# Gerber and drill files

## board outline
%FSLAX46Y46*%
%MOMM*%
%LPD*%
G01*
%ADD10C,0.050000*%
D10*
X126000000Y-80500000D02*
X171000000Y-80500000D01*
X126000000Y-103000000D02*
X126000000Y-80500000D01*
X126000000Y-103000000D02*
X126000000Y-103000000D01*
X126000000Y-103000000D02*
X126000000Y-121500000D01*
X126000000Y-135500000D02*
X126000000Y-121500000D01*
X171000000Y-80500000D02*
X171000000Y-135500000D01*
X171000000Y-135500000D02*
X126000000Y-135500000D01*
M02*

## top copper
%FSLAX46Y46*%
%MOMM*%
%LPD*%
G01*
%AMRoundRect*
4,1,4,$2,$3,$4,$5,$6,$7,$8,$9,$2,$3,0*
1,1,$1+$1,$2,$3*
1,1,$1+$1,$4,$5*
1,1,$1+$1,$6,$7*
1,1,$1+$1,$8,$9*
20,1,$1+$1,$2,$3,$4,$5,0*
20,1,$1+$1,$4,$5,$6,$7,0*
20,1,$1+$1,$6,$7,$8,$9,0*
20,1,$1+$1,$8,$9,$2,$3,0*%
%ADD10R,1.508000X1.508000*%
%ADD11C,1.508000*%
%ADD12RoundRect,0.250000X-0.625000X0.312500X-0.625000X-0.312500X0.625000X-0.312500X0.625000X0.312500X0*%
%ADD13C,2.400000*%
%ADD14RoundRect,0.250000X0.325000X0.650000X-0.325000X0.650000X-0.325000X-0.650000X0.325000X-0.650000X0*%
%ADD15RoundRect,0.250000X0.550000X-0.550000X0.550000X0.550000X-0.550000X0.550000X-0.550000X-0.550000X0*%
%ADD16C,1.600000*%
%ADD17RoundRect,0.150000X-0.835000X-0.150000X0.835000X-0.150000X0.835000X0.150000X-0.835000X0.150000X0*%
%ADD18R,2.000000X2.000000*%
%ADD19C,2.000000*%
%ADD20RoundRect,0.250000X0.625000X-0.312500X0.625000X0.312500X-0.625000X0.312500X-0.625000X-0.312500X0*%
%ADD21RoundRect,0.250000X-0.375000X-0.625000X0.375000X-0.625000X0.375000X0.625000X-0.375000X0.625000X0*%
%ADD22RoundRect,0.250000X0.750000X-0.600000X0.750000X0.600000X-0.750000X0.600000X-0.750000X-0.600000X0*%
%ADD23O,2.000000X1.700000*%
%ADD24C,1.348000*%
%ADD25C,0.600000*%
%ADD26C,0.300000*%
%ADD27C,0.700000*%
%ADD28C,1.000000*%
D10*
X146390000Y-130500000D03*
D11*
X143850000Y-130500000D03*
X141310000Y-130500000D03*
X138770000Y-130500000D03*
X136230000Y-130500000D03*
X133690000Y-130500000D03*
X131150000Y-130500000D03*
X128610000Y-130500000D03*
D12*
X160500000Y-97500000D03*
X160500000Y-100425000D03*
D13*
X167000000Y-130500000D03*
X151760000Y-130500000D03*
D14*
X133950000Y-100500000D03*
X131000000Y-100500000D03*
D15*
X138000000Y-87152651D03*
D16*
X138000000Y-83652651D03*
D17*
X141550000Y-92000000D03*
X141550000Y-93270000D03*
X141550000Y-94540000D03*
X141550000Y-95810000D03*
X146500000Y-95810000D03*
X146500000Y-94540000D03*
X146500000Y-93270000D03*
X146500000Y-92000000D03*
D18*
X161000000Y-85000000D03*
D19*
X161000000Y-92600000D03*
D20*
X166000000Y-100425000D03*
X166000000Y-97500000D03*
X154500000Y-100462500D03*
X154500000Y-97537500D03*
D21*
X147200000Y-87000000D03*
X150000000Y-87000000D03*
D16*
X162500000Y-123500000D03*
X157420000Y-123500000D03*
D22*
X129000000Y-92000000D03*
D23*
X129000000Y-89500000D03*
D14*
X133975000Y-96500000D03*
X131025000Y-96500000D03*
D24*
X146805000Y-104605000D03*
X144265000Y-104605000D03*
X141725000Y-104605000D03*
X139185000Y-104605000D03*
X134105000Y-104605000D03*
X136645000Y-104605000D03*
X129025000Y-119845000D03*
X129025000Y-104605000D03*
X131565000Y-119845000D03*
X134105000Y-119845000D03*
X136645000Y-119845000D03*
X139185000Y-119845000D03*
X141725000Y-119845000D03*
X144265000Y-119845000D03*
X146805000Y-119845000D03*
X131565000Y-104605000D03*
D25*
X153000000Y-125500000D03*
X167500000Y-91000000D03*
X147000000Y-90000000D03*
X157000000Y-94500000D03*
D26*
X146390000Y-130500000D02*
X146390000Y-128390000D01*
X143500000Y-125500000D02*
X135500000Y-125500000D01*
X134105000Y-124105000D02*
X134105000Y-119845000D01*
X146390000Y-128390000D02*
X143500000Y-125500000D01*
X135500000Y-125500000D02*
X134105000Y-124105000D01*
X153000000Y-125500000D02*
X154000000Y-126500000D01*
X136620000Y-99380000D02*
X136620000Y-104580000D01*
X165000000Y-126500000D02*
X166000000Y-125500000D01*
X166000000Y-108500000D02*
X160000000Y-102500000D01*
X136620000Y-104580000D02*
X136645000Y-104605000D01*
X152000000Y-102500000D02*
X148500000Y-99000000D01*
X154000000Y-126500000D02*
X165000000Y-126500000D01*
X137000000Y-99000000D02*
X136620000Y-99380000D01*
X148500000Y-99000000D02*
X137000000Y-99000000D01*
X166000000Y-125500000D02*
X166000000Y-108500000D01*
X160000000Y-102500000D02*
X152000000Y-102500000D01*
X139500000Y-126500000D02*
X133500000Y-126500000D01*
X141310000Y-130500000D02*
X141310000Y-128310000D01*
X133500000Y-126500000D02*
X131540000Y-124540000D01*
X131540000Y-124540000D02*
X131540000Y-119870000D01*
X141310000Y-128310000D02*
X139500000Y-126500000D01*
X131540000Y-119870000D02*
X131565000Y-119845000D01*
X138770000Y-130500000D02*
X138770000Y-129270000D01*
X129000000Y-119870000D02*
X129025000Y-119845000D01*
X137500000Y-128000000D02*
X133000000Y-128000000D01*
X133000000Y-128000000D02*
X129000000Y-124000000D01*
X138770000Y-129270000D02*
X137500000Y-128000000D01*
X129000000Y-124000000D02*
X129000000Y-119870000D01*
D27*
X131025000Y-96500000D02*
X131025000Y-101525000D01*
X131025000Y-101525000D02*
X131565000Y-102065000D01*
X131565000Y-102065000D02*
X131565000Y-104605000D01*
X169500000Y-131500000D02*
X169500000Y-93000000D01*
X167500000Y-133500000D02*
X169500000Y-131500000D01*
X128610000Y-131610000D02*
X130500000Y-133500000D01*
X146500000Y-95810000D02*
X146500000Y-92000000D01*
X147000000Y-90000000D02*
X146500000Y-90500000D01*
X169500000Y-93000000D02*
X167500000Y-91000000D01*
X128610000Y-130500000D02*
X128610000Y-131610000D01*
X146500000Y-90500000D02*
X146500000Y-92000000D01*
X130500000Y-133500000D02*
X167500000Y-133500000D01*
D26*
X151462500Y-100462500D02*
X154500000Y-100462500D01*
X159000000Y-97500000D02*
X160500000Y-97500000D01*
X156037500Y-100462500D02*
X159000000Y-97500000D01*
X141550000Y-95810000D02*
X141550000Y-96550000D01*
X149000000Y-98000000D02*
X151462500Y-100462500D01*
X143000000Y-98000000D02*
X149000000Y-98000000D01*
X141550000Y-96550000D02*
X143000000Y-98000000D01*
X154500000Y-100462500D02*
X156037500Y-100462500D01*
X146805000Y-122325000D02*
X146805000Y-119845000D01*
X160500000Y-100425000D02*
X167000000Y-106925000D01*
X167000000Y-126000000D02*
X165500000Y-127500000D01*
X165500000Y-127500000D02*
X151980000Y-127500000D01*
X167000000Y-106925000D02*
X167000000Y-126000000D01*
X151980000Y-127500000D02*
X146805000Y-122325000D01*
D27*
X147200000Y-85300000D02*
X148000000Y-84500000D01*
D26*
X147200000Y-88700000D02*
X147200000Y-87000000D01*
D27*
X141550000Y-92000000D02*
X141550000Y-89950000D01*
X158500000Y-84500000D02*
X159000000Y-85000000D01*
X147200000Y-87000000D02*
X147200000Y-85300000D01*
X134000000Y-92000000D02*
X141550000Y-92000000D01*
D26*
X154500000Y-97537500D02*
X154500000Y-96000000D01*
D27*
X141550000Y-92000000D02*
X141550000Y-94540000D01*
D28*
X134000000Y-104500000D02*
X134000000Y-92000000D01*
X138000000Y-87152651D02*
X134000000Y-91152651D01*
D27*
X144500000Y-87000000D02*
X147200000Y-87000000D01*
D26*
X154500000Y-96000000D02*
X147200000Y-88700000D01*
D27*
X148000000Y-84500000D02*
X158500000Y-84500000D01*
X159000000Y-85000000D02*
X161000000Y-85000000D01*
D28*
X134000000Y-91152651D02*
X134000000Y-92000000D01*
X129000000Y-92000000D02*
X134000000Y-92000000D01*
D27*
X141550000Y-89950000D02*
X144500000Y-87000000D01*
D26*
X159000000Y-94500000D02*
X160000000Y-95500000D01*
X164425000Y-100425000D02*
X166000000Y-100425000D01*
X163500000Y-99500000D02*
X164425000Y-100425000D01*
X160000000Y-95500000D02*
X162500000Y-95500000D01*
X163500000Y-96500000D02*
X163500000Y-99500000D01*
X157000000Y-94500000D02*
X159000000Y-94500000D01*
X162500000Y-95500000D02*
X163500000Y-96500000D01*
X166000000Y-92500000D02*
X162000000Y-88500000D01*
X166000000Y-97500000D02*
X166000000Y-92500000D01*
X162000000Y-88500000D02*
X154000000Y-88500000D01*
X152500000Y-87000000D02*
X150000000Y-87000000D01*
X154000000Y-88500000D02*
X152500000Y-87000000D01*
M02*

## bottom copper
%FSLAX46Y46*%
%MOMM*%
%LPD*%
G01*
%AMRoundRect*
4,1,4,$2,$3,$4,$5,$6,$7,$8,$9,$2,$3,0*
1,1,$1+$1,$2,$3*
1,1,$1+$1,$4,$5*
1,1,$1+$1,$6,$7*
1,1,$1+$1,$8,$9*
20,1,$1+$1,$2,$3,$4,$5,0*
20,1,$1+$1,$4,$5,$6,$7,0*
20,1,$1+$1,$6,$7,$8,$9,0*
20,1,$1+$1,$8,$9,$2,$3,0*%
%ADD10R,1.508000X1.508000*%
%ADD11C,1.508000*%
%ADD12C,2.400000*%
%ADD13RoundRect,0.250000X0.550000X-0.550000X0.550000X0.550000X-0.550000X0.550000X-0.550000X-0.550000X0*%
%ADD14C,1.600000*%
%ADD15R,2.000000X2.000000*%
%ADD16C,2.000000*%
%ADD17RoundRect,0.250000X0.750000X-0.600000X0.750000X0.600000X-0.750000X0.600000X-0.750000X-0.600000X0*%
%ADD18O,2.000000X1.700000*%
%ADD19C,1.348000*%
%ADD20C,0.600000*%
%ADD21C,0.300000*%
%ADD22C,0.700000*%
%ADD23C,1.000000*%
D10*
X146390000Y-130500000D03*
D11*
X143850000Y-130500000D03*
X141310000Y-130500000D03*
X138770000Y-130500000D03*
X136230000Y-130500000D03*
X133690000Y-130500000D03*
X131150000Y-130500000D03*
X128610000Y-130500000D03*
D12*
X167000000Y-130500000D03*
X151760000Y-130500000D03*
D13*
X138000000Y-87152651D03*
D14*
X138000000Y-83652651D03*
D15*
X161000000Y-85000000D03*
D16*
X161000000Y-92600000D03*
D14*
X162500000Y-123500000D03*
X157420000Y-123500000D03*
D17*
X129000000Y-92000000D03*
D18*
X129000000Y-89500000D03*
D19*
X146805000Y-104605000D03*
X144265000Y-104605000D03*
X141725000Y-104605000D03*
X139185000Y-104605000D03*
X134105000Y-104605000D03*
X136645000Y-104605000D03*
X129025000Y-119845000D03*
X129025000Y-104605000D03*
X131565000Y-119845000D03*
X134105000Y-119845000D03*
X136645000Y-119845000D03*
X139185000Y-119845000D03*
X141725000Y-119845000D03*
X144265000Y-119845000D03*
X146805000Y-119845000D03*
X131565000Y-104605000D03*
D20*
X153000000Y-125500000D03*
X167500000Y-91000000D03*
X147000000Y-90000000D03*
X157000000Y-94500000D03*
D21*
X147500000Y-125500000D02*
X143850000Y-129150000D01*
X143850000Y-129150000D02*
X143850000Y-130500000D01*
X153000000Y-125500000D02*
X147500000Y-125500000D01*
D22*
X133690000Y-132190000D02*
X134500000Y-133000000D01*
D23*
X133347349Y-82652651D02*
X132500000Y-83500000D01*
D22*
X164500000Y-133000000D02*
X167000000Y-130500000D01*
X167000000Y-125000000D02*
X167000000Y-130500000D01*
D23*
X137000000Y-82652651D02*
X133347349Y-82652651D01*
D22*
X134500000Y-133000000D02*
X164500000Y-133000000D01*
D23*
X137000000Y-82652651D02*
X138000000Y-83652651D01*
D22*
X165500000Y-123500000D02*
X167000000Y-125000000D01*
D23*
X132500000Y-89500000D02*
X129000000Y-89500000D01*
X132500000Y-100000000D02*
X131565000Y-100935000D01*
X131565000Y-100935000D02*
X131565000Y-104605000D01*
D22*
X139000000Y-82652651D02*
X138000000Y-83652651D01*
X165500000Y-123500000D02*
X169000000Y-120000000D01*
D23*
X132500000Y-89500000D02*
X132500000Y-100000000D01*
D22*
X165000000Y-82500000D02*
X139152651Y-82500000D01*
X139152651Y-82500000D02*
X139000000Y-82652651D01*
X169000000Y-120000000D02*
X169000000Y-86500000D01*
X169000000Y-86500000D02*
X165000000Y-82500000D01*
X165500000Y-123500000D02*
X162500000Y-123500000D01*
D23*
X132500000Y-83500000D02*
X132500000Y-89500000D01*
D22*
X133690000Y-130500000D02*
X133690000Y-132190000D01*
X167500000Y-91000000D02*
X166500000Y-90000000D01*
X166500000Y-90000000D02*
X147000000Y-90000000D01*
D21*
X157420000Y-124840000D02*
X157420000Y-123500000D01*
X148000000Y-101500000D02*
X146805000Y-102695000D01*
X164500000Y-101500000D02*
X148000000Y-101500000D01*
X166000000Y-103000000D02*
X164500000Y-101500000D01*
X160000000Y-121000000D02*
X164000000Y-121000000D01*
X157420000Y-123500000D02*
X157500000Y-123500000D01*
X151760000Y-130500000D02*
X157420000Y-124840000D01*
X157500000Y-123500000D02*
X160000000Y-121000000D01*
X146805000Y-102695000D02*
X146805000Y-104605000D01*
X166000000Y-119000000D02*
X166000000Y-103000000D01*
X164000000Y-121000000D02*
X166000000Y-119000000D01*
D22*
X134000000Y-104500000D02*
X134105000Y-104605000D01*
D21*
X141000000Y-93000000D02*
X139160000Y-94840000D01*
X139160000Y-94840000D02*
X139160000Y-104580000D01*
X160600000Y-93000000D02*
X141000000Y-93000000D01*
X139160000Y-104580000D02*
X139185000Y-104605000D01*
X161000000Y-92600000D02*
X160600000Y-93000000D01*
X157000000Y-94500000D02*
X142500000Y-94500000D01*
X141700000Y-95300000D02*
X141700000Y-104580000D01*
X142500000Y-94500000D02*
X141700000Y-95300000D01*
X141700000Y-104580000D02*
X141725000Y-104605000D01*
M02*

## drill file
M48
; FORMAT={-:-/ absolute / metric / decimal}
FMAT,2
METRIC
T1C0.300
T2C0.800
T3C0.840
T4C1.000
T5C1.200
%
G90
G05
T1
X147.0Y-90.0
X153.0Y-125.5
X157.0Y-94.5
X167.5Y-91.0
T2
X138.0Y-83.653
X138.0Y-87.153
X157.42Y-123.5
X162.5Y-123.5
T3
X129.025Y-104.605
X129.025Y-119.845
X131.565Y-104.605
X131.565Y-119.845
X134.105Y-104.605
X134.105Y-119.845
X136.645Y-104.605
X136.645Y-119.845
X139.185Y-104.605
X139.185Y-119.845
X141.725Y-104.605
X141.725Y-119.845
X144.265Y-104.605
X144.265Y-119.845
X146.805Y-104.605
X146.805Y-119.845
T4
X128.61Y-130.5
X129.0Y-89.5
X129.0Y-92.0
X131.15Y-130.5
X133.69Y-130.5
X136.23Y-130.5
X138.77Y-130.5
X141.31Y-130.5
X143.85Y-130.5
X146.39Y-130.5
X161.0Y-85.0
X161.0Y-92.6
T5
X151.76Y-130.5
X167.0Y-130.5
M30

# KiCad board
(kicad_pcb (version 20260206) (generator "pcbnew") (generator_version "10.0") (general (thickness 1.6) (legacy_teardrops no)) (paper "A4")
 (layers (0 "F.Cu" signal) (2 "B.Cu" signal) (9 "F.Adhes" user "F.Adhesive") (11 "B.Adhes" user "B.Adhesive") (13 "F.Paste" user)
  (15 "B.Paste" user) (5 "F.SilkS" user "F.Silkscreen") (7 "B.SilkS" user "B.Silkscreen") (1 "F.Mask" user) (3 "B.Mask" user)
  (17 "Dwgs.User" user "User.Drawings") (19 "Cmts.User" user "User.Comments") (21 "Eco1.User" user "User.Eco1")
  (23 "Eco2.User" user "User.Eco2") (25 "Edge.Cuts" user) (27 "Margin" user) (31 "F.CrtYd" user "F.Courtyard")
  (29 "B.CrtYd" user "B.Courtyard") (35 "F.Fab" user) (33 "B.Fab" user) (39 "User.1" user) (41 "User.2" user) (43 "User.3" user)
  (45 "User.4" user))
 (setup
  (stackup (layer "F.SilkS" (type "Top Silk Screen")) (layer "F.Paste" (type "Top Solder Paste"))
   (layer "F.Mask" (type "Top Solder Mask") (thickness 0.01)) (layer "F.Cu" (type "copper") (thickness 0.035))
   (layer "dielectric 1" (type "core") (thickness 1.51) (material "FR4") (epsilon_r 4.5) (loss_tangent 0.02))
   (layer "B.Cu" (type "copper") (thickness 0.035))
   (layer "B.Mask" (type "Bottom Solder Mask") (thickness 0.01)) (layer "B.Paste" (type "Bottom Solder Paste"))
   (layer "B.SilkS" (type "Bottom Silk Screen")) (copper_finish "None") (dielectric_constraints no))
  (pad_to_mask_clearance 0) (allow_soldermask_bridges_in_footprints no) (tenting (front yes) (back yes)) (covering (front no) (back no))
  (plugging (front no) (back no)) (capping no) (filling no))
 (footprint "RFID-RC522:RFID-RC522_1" (layer "F.Cu") (at 137.5 130.5 180)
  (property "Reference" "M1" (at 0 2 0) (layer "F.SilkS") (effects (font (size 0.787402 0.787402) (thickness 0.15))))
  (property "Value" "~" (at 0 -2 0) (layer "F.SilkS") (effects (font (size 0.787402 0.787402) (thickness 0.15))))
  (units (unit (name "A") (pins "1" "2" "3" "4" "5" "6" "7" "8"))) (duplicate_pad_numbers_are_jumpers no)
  (pad "1" thru_hole rect (at -8.89 0 180) (size 1.508 1.508) (drill 1) (layers "*.Cu" "*.Mask") (remove_unused_layers no)
   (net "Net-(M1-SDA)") (solder_mask_margin 0.102))
  (pad "2" thru_hole circle (at -6.35 0 180) (size 1.508 1.508) (drill 1) (layers "*.Cu" "*.Mask") (remove_unused_layers no)
   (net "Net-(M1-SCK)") (solder_mask_margin 0.102))
  (pad "3" thru_hole circle (at -3.81 0 180) (size 1.508 1.508) (drill 1) (layers "*.Cu" "*.Mask") (remove_unused_layers no)
   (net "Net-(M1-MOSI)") (solder_mask_margin 0.102))
  (pad "4" thru_hole circle (at -1.27 0 180) (size 1.508 1.508) (drill 1) (layers "*.Cu" "*.Mask") (remove_unused_layers no)
   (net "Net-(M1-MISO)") (solder_mask_margin 0.102))
  (pad "5" thru_hole circle (at 1.27 0 180) (size 1.508 1.508) (drill 1) (layers "*.Cu" "*.Mask") (remove_unused_layers no)
   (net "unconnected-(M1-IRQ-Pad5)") (solder_mask_margin 0.102))
  (pad "6" thru_hole circle (at 3.81 0 180) (size 1.508 1.508) (drill 1) (layers "*.Cu" "*.Mask") (remove_unused_layers no) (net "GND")
   (solder_mask_margin 0.102))
  (pad "7" thru_hole circle (at 6.35 0 180) (size 1.508 1.508) (drill 1) (layers "*.Cu" "*.Mask") (remove_unused_layers no)
   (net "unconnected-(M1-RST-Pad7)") (solder_mask_margin 0.102))
  (pad "8" thru_hole circle (at 8.89 0 180) (size 1.508 1.508) (drill 1) (layers "*.Cu" "*.Mask") (remove_unused_layers no) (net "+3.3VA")
   (solder_mask_margin 0.102)))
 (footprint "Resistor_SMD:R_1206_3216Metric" (layer "F.Cu") (at 160.5 98.9625 -90)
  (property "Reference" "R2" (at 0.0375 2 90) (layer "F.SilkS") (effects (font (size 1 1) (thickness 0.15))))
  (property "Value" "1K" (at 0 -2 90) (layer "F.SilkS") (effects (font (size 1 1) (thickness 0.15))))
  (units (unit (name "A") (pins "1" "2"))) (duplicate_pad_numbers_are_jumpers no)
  (pad "1" smd roundrect (at -1.4625 0 270) (size 1.125 1.75) (layers "F.Cu" "F.Mask" "F.Paste") (roundrect_rratio 0.222222)
   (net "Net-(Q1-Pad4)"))
  (pad "2" smd roundrect (at 1.4625 0 270) (size 1.125 1.75) (layers "F.Cu" "F.Mask" "F.Paste") (roundrect_rratio 0.222222)
   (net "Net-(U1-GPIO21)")))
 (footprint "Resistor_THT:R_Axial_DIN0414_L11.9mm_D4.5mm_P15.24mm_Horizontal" (layer "F.Cu") (at 167 130.5 180)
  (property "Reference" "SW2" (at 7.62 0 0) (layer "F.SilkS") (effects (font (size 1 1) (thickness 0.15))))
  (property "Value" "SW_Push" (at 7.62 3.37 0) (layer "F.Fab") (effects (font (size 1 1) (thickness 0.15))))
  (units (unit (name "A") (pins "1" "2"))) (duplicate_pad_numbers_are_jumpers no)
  (pad "1" thru_hole circle (at 0 0 180) (size 2.4 2.4) (drill 1.2) (layers "*.Cu" "*.Mask") (remove_unused_layers no) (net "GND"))
  (pad "2" thru_hole circle (at 15.24 0 180) (size 2.4 2.4) (drill 1.2) (layers "*.Cu" "*.Mask") (remove_unused_layers no)
   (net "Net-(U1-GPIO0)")))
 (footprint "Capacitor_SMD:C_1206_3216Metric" (layer "F.Cu") (at 132.475 100.5 180)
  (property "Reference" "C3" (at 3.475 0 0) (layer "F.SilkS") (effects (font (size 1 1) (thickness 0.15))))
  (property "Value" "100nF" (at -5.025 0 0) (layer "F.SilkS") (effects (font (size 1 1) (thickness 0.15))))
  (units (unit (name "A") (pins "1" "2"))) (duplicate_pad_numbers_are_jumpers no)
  (pad "1" smd roundrect (at -1.475 0 180) (size 1.15 1.8) (layers "F.Cu" "F.Mask" "F.Paste") (roundrect_rratio 0.217391) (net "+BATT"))
  (pad "2" smd roundrect (at 1.475 0 180) (size 1.15 1.8) (layers "F.Cu" "F.Mask" "F.Paste") (roundrect_rratio 0.217391) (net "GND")))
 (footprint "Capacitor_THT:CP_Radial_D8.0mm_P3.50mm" (layer "F.Cu") (at 138 87.152651 90)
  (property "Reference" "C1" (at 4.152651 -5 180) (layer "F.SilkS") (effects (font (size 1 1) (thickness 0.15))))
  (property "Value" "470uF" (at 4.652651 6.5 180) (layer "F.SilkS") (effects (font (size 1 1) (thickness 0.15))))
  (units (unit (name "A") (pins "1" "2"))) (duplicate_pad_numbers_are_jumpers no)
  (pad "1" thru_hole roundrect (at 0 0 90) (size 1.6 1.6) (drill 0.8) (layers "*.Cu" "*.Mask") (remove_unused_layers no)
   (roundrect_rratio 0.15625) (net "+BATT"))
  (pad "2" thru_hole circle (at 3.5 0 90) (size 1.6 1.6) (drill 0.8) (layers "*.Cu" "*.Mask") (remove_unused_layers no) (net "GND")))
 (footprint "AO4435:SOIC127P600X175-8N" (layer "F.Cu") (at 144.025 93.905)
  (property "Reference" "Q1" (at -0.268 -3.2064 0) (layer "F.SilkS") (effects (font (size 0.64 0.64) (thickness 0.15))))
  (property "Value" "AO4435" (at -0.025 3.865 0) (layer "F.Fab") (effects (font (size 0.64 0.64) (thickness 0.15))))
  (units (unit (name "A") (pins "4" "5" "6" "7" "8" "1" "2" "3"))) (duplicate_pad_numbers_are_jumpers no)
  (pad "1" smd roundrect (at -2.475 -1.905) (size 1.97 0.6) (layers "F.Cu" "F.Mask" "F.Paste") (roundrect_rratio 0.25) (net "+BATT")
   (solder_mask_margin 0.102))
  (pad "2" smd roundrect (at -2.475 -0.635) (size 1.97 0.6) (layers "F.Cu" "F.Mask" "F.Paste") (roundrect_rratio 0.25) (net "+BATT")
   (solder_mask_margin 0.102))
  (pad "3" smd roundrect (at -2.475 0.635) (size 1.97 0.6) (layers "F.Cu" "F.Mask" "F.Paste") (roundrect_rratio 0.25) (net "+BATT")
   (solder_mask_margin 0.102))
  (pad "4" smd roundrect (at -2.475 1.905) (size 1.97 0.6) (layers "F.Cu" "F.Mask" "F.Paste") (roundrect_rratio 0.25) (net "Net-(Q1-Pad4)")
   (solder_mask_margin 0.102))
  (pad "5" smd roundrect (at 2.475 1.905) (size 1.97 0.6) (layers "F.Cu" "F.Mask" "F.Paste") (roundrect_rratio 0.25) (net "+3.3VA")
   (solder_mask_margin 0.102))
  (pad "6" smd roundrect (at 2.475 0.635) (size 1.97 0.6) (layers "F.Cu" "F.Mask" "F.Paste") (roundrect_rratio 0.25) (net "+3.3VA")
   (solder_mask_margin 0.102))
  (pad "7" smd roundrect (at 2.475 -0.635) (size 1.97 0.6) (layers "F.Cu" "F.Mask" "F.Paste") (roundrect_rratio 0.25) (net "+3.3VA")
   (solder_mask_margin 0.102))
  (pad "8" smd roundrect (at 2.475 -1.905) (size 1.97 0.6) (layers "F.Cu" "F.Mask" "F.Paste") (roundrect_rratio 0.25) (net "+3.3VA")
   (solder_mask_margin 0.102)))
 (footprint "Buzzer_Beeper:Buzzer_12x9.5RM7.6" (layer "F.Cu") (at 161 85 -90)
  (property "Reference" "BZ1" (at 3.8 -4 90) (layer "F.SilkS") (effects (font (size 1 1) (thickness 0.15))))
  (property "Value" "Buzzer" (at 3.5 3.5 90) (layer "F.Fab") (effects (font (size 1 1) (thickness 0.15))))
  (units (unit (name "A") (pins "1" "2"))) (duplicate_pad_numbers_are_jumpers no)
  (pad "1" thru_hole rect (at 0 0 270) (size 2 2) (drill 1) (layers "*.Cu" "*.Mask") (remove_unused_layers no) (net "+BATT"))
  (pad "2" thru_hole circle (at 7.6 0 270) (size 2 2) (drill 1) (layers "*.Cu" "*.Mask") (remove_unused_layers no) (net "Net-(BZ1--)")))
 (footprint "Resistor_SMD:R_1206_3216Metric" (layer "F.Cu") (at 166 98.9625 90)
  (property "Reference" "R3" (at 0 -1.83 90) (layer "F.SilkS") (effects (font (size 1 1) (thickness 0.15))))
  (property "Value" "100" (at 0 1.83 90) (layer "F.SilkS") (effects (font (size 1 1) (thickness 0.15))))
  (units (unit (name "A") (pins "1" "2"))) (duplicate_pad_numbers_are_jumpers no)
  (pad "1" smd roundrect (at -1.4625 0 90) (size 1.125 1.75) (layers "F.Cu" "F.Mask" "F.Paste") (roundrect_rratio 0.222222)
   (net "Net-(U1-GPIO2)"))
  (pad "2" smd roundrect (at 1.4625 0 90) (size 1.125 1.75) (layers "F.Cu" "F.Mask" "F.Paste") (roundrect_rratio 0.222222)
   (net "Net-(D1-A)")))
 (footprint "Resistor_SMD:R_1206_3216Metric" (layer "F.Cu") (at 154.5 99 90)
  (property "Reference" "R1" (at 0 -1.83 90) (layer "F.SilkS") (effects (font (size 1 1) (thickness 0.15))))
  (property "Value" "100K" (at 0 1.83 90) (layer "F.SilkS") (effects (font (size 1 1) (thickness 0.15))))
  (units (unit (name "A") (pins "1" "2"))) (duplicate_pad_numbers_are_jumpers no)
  (pad "1" smd roundrect (at -1.4625 0 90) (size 1.125 1.75) (layers "F.Cu" "F.Mask" "F.Paste") (roundrect_rratio 0.222222)
   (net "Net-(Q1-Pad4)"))
  (pad "2" smd roundrect (at 1.4625 0 90) (size 1.125 1.75) (layers "F.Cu" "F.Mask" "F.Paste") (roundrect_rratio 0.222222) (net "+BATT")))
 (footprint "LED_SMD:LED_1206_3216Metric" (layer "F.Cu") (at 148.6 87)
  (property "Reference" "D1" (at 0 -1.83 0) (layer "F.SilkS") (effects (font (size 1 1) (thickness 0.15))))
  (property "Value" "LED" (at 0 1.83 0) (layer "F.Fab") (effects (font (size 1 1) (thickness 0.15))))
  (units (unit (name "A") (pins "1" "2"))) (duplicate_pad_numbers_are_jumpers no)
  (pad "1" smd roundrect (at -1.4 0) (size 1.25 1.75) (layers "F.Cu" "F.Mask" "F.Paste") (roundrect_rratio 0.2) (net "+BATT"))
  (pad "2" smd roundrect (at 1.4 0) (size 1.25 1.75) (layers "F.Cu" "F.Mask" "F.Paste") (roundrect_rratio 0.2) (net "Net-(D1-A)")))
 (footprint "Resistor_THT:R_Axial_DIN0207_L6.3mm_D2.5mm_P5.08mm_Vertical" (layer "F.Cu") (at 162.5 123.5 180)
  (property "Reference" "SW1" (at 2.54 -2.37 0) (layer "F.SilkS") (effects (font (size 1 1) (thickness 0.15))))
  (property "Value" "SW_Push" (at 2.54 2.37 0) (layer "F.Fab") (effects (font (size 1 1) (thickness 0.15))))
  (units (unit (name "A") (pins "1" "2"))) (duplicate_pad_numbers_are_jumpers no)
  (pad "1" thru_hole circle (at 0 0 180) (size 1.6 1.6) (drill 0.8) (layers "*.Cu" "*.Mask") (remove_unused_layers no) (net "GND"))
  (pad "2" thru_hole circle (at 5.08 0 180) (size 1.6 1.6) (drill 0.8) (layers "*.Cu" "*.Mask") (remove_unused_layers no)
   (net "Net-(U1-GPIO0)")))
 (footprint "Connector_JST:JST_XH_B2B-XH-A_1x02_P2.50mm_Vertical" (layer "F.Cu") (at 129 92 90)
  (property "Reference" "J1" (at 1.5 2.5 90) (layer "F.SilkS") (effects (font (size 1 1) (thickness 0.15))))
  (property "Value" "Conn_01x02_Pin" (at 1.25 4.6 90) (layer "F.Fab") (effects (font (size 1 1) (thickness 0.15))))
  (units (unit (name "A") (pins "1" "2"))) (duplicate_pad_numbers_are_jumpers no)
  (pad "1" thru_hole roundrect (at 0 0 90) (size 1.7 2) (drill 1) (layers "*.Cu" "*.Mask") (remove_unused_layers no)
   (roundrect_rratio 0.147059) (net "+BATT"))
  (pad "2" thru_hole oval (at 2.5 0 90) (size 1.7 2) (drill 1) (layers "*.Cu" "*.Mask") (remove_unused_layers no) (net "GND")))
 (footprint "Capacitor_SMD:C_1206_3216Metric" (layer "F.Cu") (at 132.5 96.5 180)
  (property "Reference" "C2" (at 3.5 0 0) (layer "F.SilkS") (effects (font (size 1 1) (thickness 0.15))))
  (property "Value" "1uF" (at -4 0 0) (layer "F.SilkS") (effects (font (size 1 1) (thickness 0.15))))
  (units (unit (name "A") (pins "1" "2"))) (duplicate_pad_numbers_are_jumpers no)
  (pad "1" smd roundrect (at -1.475 0 180) (size 1.15 1.8) (layers "F.Cu" "F.Mask" "F.Paste") (roundrect_rratio 0.217391) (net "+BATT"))
  (pad "2" smd roundrect (at 1.475 0 180) (size 1.15 1.8) (layers "F.Cu" "F.Mask" "F.Paste") (roundrect_rratio 0.217391) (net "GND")))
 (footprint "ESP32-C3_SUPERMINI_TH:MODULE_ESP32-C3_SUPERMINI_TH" (layer "F.Cu") (at 138.925 112.225 90)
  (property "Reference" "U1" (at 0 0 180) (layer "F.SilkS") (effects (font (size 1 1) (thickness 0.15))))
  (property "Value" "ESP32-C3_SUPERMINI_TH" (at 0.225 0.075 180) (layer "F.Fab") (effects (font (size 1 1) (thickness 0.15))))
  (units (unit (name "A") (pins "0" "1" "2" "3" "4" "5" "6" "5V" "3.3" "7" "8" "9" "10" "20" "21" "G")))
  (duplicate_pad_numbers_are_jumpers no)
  (pad "0" thru_hole circle (at 7.62 7.88 90) (size 1.348 1.348) (drill 0.84) (layers "*.Cu" "*.Mask") (remove_unused_layers no)
   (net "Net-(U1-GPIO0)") (solder_mask_margin 0.102))
  (pad "1" thru_hole circle (at 7.62 5.34 90) (size 1.348 1.348) (drill 0.84) (layers "*.Cu" "*.Mask") (remove_unused_layers no)
   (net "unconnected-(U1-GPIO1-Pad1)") (solder_mask_margin 0.102))
  (pad "2" thru_hole circle (at 7.62 2.8 90) (size 1.348 1.348) (drill 0.84) (layers "*.Cu" "*.Mask") (remove_unused_layers no)
   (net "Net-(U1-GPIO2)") (solder_mask_margin 0.102))
  (pad "3" thru_hole circle (at 7.62 0.26 90) (size 1.348 1.348) (drill 0.84) (layers "*.Cu" "*.Mask") (remove_unused_layers no)
   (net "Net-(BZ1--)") (solder_mask_margin 0.102))
  (pad "3.3" thru_hole circle (at 7.62 -4.82 90) (size 1.348 1.348) (drill 0.84) (layers "*.Cu" "*.Mask") (remove_unused_layers no)
   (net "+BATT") (solder_mask_margin 0.102))
  (pad "4" thru_hole circle (at 7.62 -2.28 90) (size 1.348 1.348) (drill 0.84) (layers "*.Cu" "*.Mask") (remove_unused_layers no)
   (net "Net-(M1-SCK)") (solder_mask_margin 0.102))
  (pad "5" thru_hole circle (at -7.62 -9.9 90) (size 1.348 1.348) (drill 0.84) (layers "*.Cu" "*.Mask") (remove_unused_layers no)
   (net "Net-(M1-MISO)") (solder_mask_margin 0.102))
  (pad "5V" thru_hole circle (at 7.62 -9.9 90) (size 1.348 1.348) (drill 0.84) (layers "*.Cu" "*.Mask") (remove_unused_layers no)
   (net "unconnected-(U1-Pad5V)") (solder_mask_margin 0.102))
  (pad "6" thru_hole circle (at -7.62 -7.36 90) (size 1.348 1.348) (drill 0.84) (layers "*.Cu" "*.Mask") (remove_unused_layers no)
   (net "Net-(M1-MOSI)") (solder_mask_margin 0.102))
  (pad "7" thru_hole circle (at -7.62 -4.82 90) (size 1.348 1.348) (drill 0.84) (layers "*.Cu" "*.Mask") (remove_unused_layers no)
   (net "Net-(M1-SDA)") (solder_mask_margin 0.102))
  (pad "8" thru_hole circle (at -7.62 -2.28 90) (size 1.348 1.348) (drill 0.84) (layers "*.Cu" "*.Mask") (remove_unused_layers no)
   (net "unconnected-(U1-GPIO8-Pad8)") (solder_mask_margin 0.102))
  (pad "9" thru_hole circle (at -7.62 0.26 90) (size 1.348 1.348) (drill 0.84) (layers "*.Cu" "*.Mask") (remove_unused_layers no)
   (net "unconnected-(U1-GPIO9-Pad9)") (solder_mask_margin 0.102))
  (pad "10" thru_hole circle (at -7.62 2.8 90) (size 1.348 1.348) (drill 0.84) (layers "*.Cu" "*.Mask") (remove_unused_layers no)
   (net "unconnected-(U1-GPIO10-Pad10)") (solder_mask_margin 0.102))
  (pad "20" thru_hole circle (at -7.62 5.34 90) (size 1.348 1.348) (drill 0.84) (layers "*.Cu" "*.Mask") (remove_unused_layers no)
   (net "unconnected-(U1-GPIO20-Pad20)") (solder_mask_margin 0.102))
  (pad "21" thru_hole circle (at -7.62 7.88 90) (size 1.348 1.348) (drill 0.84) (layers "*.Cu" "*.Mask") (remove_unused_layers no)
   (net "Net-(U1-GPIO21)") (solder_mask_margin 0.102))
  (pad "G" thru_hole circle (at 7.62 -7.36 90) (size 1.348 1.348) (drill 0.84) (layers "*.Cu" "*.Mask") (remove_unused_layers no)
   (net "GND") (solder_mask_margin 0.102)))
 (gr_line (start 126 80.5) (end 171 80.5) (stroke (width 0.05) (type default)) (layer "Edge.Cuts"))
 (gr_line (start 126 103) (end 126 80.5) (stroke (width 0.05) (type default)) (layer "Edge.Cuts"))
 (gr_line (start 126 103) (end 126 103) (stroke (width 0.05) (type default)) (layer "Edge.Cuts"))
 (gr_line (start 126 103) (end 126 121.5) (stroke (width 0.05) (type default)) (layer "Edge.Cuts"))
 (gr_line (start 126 135.5) (end 126 121.5) (stroke (width 0.05) (type default)) (layer "Edge.Cuts"))
 (gr_line (start 171 80.5) (end 171 135.5) (stroke (width 0.05) (type default)) (layer "Edge.Cuts"))
 (gr_line (start 171 135.5) (end 126 135.5) (stroke (width 0.05) (type default)) (layer "Edge.Cuts"))
 (segment (start 146.39 130.5) (end 146.39 128.39) (width 0.3) (layer "F.Cu") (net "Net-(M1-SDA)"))
 (segment (start 143.5 125.5) (end 135.5 125.5) (width 0.3) (layer "F.Cu") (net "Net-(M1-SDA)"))
 (segment (start 134.105 124.105) (end 134.105 119.845) (width 0.3) (layer "F.Cu") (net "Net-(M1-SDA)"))
 (segment (start 146.39 128.39) (end 143.5 125.5) (width 0.3) (layer "F.Cu") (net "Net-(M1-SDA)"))
 (segment (start 135.5 125.5) (end 134.105 124.105) (width 0.3) (layer "F.Cu") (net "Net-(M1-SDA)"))
 (segment (start 153 125.5) (end 154 126.5) (width 0.3) (layer "F.Cu") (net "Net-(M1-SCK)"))
 (segment (start 136.62 99.38) (end 136.62 104.58) (width 0.3) (layer "F.Cu") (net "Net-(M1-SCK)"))
 (segment (start 165 126.5) (end 166 125.5) (width 0.3) (layer "F.Cu") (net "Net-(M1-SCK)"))
 (segment (start 166 108.5) (end 160 102.5) (width 0.3) (layer "F.Cu") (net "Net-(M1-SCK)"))
 (segment (start 136.62 104.58) (end 136.645 104.605) (width 0.3) (layer "F.Cu") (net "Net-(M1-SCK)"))
 (segment (start 152 102.5) (end 148.5 99) (width 0.3) (layer "F.Cu") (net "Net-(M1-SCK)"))
 (segment (start 154 126.5) (end 165 126.5) (width 0.3) (layer "F.Cu") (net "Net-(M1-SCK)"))
 (segment (start 137 99) (end 136.62 99.38) (width 0.3) (layer "F.Cu") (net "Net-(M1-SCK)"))
 (segment (start 148.5 99) (end 137 99) (width 0.3) (layer "F.Cu") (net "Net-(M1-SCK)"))
 (segment (start 166 125.5) (end 166 108.5) (width 0.3) (layer "F.Cu") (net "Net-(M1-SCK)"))
 (segment (start 160 102.5) (end 152 102.5) (width 0.3) (layer "F.Cu") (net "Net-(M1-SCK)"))
 (via (at 153 125.5) (size 0.6) (drill 0.3) (layers "F.Cu" "B.Cu") (capping no) (covering (front no) (back no))
  (plugging (front no) (back no)) (filling no) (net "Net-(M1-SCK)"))
 (segment (start 147.5 125.5) (end 143.85 129.15) (width 0.3) (layer "B.Cu") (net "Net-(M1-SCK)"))
 (segment (start 143.85 129.15) (end 143.85 130.5) (width 0.3) (layer "B.Cu") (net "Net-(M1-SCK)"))
 (segment (start 153 125.5) (end 147.5 125.5) (width 0.3) (layer "B.Cu") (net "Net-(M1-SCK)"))
 (segment (start 139.5 126.5) (end 133.5 126.5) (width 0.3) (layer "F.Cu") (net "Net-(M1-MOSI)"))
 (segment (start 141.31 130.5) (end 141.31 128.31) (width 0.3) (layer "F.Cu") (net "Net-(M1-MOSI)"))
 (segment (start 133.5 126.5) (end 131.54 124.54) (width 0.3) (layer "F.Cu") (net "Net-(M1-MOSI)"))
 (segment (start 131.54 124.54) (end 131.54 119.87) (width 0.3) (layer "F.Cu") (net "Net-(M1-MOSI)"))
 (segment (start 141.31 128.31) (end 139.5 126.5) (width 0.3) (layer "F.Cu") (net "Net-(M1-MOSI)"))
 (segment (start 131.54 119.87) (end 131.565 119.845) (width 0.3) (layer "F.Cu") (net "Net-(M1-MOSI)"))
 (segment (start 138.77 130.5) (end 138.77 129.27) (width 0.3) (layer "F.Cu") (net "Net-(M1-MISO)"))
 (segment (start 129 119.87) (end 129.025 119.845) (width 0.3) (layer "F.Cu") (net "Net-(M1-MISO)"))
 (segment (start 137.5 128) (end 133 128) (width 0.3) (layer "F.Cu") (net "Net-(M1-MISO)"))
 (segment (start 133 128) (end 129 124) (width 0.3) (layer "F.Cu") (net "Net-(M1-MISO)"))
 (segment (start 138.77 129.27) (end 137.5 128) (width 0.3) (layer "F.Cu") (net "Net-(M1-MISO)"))
 (segment (start 129 124) (end 129 119.87) (width 0.3) (layer "F.Cu") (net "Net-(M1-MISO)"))
 (segment (start 131.025 96.5) (end 131.025 101.525) (width 0.7) (layer "F.Cu") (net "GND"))
 (segment (start 131.025 101.525) (end 131.565 102.065) (width 0.7) (layer "F.Cu") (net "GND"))
 (segment (start 131.565 102.065) (end 131.565 104.605) (width 0.7) (layer "F.Cu") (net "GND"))
 (segment (start 133.69 132.19) (end 134.5 133) (width 0.7) (layer "B.Cu") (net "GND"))
 (segment (start 133.347349 82.652651) (end 132.5 83.5) (width 1) (layer "B.Cu") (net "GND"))
 (segment (start 164.5 133) (end 167 130.5) (width 0.7) (layer "B.Cu") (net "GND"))
 (segment (start 167 125) (end 167 130.5) (width 0.7) (layer "B.Cu") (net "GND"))
 (segment (start 137 82.652651) (end 133.347349 82.652651) (width 1) (layer "B.Cu") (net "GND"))
 (segment (start 134.5 133) (end 164.5 133) (width 0.7) (layer "B.Cu") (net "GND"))
 (segment (start 137 82.652651) (end 138 83.652651) (width 1) (layer "B.Cu") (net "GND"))
 (segment (start 165.5 123.5) (end 167 125) (width 0.7) (layer "B.Cu") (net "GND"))
 (segment (start 132.5 89.5) (end 129 89.5) (width 1) (layer "B.Cu") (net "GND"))
 (segment (start 132.5 100) (end 131.565 100.935) (width 1) (layer "B.Cu") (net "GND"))
 (segment (start 131.565 100.935) (end 131.565 104.605) (width 1) (layer "B.Cu") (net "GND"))
 (segment (start 139 82.652651) (end 138 83.652651) (width 0.7) (layer "B.Cu") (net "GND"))
 (segment (start 165.5 123.5) (end 169 120) (width 0.7) (layer "B.Cu") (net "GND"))
 (segment (start 132.5 89.5) (end 132.5 100) (width 1) (layer "B.Cu") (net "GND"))
 (segment (start 165 82.5) (end 139.152651 82.5) (width 0.7) (layer "B.Cu") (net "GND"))
 (segment (start 139.152651 82.5) (end 139 82.652651) (width 0.7) (layer "B.Cu") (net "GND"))
 (segment (start 169 120) (end 169 86.5) (width 0.7) (layer "B.Cu") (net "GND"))
 (segment (start 169 86.5) (end 165 82.5) (width 0.7) (layer "B.Cu") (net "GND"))
 (segment (start 165.5 123.5) (end 162.5 123.5) (width 0.7) (layer "B.Cu") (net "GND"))
 (segment (start 132.5 83.5) (end 132.5 89.5) (width 1) (layer "B.Cu") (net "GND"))
 (segment (start 133.69 130.5) (end 133.69 132.19) (width 0.7) (layer "B.Cu") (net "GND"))
 (segment (start 169.5 131.5) (end 169.5 93) (width 0.7) (layer "F.Cu") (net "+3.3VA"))
 (segment (start 167.5 133.5) (end 169.5 131.5) (width 0.7) (layer "F.Cu") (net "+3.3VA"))
 (segment (start 128.61 131.61) (end 130.5 133.5) (width 0.7) (layer "F.Cu") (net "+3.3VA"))
 (segment (start 146.5 95.81) (end 146.5 92) (width 0.7) (layer "F.Cu") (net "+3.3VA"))
 (segment (start 147 90) (end 146.5 90.5) (width 0.7) (layer "F.Cu") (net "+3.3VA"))
 (segment (start 169.5 93) (end 167.5 91) (width 0.7) (layer "F.Cu") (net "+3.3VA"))
 (segment (start 128.61 130.5) (end 128.61 131.61) (width 0.7) (layer "F.Cu") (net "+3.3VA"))
 (segment (start 146.5 90.5) (end 146.5 92) (width 0.7) (layer "F.Cu") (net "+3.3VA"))
 (segment (start 130.5 133.5) (end 167.5 133.5) (width 0.7) (layer "F.Cu") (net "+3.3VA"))
 (via (at 167.5 91) (size 0.6) (drill 0.3) (layers "F.Cu" "B.Cu") (capping no) (covering (front no) (back no))
  (plugging (front no) (back no)) (filling no) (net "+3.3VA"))
 (via (at 147 90) (size 0.6) (drill 0.3) (layers "F.Cu" "B.Cu") (capping no) (covering (front no) (back no)) (plugging (front no) (back no))
  (filling no) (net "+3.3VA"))
 (segment (start 167.5 91) (end 166.5 90) (width 0.7) (layer "B.Cu") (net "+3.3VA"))
 (segment (start 166.5 90) (end 147 90) (width 0.7) (layer "B.Cu") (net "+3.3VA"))
 (segment (start 151.4625 100.4625) (end 154.5 100.4625) (width 0.3) (layer "F.Cu") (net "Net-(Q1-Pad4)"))
 (segment (start 159 97.5) (end 160.5 97.5) (width 0.3) (layer "F.Cu") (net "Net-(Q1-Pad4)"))
 (segment (start 156.0375 100.4625) (end 159 97.5) (width 0.3) (layer "F.Cu") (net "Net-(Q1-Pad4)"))
 (segment (start 141.55 95.81) (end 141.55 96.55) (width 0.3) (layer "F.Cu") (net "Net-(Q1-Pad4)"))
 (segment (start 149 98) (end 151.4625 100.4625) (width 0.3) (layer "F.Cu") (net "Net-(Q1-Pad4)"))
 (segment (start 143 98) (end 149 98) (width 0.3) (layer "F.Cu") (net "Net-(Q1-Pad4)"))
 (segment (start 141.55 96.55) (end 143 98) (width 0.3) (layer "F.Cu") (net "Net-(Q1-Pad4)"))
 (segment (start 154.5 100.4625) (end 156.0375 100.4625) (width 0.3) (layer "F.Cu") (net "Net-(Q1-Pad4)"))
 (segment (start 146.805 122.325) (end 146.805 119.845) (width 0.3) (layer "F.Cu") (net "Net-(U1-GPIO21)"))
 (segment (start 160.5 100.425) (end 167 106.925) (width 0.3) (layer "F.Cu") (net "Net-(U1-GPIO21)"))
 (segment (start 167 126) (end 165.5 127.5) (width 0.3) (layer "F.Cu") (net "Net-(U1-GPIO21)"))
 (segment (start 165.5 127.5) (end 151.98 127.5) (width 0.3) (layer "F.Cu") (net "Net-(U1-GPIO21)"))
 (segment (start 167 106.925) (end 167 126) (width 0.3) (layer "F.Cu") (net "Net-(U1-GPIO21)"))
 (segment (start 151.98 127.5) (end 146.805 122.325) (width 0.3) (layer "F.Cu") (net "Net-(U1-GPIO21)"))
 (segment (start 157.42 124.84) (end 157.42 123.5) (width 0.3) (layer "B.Cu") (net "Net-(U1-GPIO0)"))
 (segment (start 148 101.5) (end 146.805 102.695) (width 0.3) (layer "B.Cu") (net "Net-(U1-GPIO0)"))
 (segment (start 164.5 101.5) (end 148 101.5) (width 0.3) (layer "B.Cu") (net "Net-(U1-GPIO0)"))
 (segment (start 166 103) (end 164.5 101.5) (width 0.3) (layer "B.Cu") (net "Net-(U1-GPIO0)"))
 (segment (start 160 121) (end 164 121) (width 0.3) (layer "B.Cu") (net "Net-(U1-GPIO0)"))
 (segment (start 157.42 123.5) (end 157.5 123.5) (width 0.3) (layer "B.Cu") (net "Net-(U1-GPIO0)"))
 (segment (start 151.76 130.5) (end 157.42 124.84) (width 0.3) (layer "B.Cu") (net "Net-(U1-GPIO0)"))
 (segment (start 157.5 123.5) (end 160 121) (width 0.3) (layer "B.Cu") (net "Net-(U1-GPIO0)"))
 (segment (start 146.805 102.695) (end 146.805 104.605) (width 0.3) (layer "B.Cu") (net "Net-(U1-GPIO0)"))
 (segment (start 166 119) (end 166 103) (width 0.3) (layer "B.Cu") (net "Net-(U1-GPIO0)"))
 (segment (start 164 121) (end 166 119) (width 0.3) (layer "B.Cu") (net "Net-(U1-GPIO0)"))
 (segment (start 147.2 85.3) (end 148 84.5) (width 0.7) (layer "F.Cu") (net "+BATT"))
 (segment (start 147.2 88.7) (end 147.2 87) (width 0.3) (layer "F.Cu") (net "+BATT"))
 (segment (start 141.55 92) (end 141.55 89.95) (width 0.7) (layer "F.Cu") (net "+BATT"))
 (segment (start 158.5 84.5) (end 159 85) (width 0.7) (layer "F.Cu") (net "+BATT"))
 (segment (start 147.2 87) (end 147.2 85.3) (width 0.7) (layer "F.Cu") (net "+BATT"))
 (segment (start 134 92) (end 141.55 92) (width 0.7) (layer "F.Cu") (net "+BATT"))
 (segment (start 154.5 97.5375) (end 154.5 96) (width 0.3) (layer "F.Cu") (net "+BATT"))
 (segment (start 141.55 92) (end 141.55 94.54) (width 0.7) (layer "F.Cu") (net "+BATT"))
 (segment (start 134 104.5) (end 134 92) (width 1) (layer "F.Cu") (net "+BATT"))
 (segment (start 138 87.152651) (end 134 91.152651) (width 1) (layer "F.Cu") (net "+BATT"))
 (segment (start 144.5 87) (end 147.2 87) (width 0.7) (layer "F.Cu") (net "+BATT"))
 (segment (start 154.5 96) (end 147.2 88.7) (width 0.3) (layer "F.Cu") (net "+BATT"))
 (segment (start 148 84.5) (end 158.5 84.5) (width 0.7) (layer "F.Cu") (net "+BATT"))
 (segment (start 159 85) (end 161 85) (width 0.7) (layer "F.Cu") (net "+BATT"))
 (segment (start 134 91.152651) (end 134 92) (width 1) (layer "F.Cu") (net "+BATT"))
 (segment (start 129 92) (end 134 92) (width 1) (layer "F.Cu") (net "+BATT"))
 (segment (start 141.55 89.95) (end 144.5 87) (width 0.7) (layer "F.Cu") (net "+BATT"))
 (segment (start 134 104.5) (end 134.105 104.605) (width 0.7) (layer "B.Cu") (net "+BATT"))
 (segment (start 141 93) (end 139.16 94.84) (width 0.3) (layer "B.Cu") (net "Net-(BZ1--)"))
 (segment (start 139.16 94.84) (end 139.16 104.58) (width 0.3) (layer "B.Cu") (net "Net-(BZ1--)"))
 (segment (start 160.6 93) (end 141 93) (width 0.3) (layer "B.Cu") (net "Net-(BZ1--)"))
 (segment (start 139.16 104.58) (end 139.185 104.605) (width 0.3) (layer "B.Cu") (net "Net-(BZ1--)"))
 (segment (start 161 92.6) (end 160.6 93) (width 0.3) (layer "B.Cu") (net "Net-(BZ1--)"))
 (segment (start 159 94.5) (end 160 95.5) (width 0.3) (layer "F.Cu") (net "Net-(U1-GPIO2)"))
 (segment (start 164.425 100.425) (end 166 100.425) (width 0.3) (layer "F.Cu") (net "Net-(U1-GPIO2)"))
 (segment (start 163.5 99.5) (end 164.425 100.425) (width 0.3) (layer "F.Cu") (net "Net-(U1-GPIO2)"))
 (segment (start 160 95.5) (end 162.5 95.5) (width 0.3) (layer "F.Cu") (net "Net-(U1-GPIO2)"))
 (segment (start 163.5 96.5) (end 163.5 99.5) (width 0.3) (layer "F.Cu") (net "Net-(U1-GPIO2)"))
 (segment (start 157 94.5) (end 159 94.5) (width 0.3) (layer "F.Cu") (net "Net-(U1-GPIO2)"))
 (segment (start 162.5 95.5) (end 163.5 96.5) (width 0.3) (layer "F.Cu") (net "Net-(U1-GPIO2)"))
 (via (at 157 94.5) (size 0.6) (drill 0.3) (layers "F.Cu" "B.Cu") (capping no) (covering (front no) (back no))
  (plugging (front no) (back no)) (filling no) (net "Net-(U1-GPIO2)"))
 (segment (start 157 94.5) (end 142.5 94.5) (width 0.3) (layer "B.Cu") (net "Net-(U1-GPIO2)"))
 (segment (start 141.7 95.3) (end 141.7 104.58) (width 0.3) (layer "B.Cu") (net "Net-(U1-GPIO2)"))
 (segment (start 142.5 94.5) (end 141.7 95.3) (width 0.3) (layer "B.Cu") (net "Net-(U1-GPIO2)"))
 (segment (start 141.7 104.58) (end 141.725 104.605) (width 0.3) (layer "B.Cu") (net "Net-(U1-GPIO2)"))
 (segment (start 166 92.5) (end 162 88.5) (width 0.3) (layer "F.Cu") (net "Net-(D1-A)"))
 (segment (start 166 97.5) (end 166 92.5) (width 0.3) (layer "F.Cu") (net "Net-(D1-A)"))
 (segment (start 162 88.5) (end 154 88.5) (width 0.3) (layer "F.Cu") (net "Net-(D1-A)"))
 (segment (start 152.5 87) (end 150 87) (width 0.3) (layer "F.Cu") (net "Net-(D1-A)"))
 (segment (start 154 88.5) (end 152.5 87) (width 0.3) (layer "F.Cu") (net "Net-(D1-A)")))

